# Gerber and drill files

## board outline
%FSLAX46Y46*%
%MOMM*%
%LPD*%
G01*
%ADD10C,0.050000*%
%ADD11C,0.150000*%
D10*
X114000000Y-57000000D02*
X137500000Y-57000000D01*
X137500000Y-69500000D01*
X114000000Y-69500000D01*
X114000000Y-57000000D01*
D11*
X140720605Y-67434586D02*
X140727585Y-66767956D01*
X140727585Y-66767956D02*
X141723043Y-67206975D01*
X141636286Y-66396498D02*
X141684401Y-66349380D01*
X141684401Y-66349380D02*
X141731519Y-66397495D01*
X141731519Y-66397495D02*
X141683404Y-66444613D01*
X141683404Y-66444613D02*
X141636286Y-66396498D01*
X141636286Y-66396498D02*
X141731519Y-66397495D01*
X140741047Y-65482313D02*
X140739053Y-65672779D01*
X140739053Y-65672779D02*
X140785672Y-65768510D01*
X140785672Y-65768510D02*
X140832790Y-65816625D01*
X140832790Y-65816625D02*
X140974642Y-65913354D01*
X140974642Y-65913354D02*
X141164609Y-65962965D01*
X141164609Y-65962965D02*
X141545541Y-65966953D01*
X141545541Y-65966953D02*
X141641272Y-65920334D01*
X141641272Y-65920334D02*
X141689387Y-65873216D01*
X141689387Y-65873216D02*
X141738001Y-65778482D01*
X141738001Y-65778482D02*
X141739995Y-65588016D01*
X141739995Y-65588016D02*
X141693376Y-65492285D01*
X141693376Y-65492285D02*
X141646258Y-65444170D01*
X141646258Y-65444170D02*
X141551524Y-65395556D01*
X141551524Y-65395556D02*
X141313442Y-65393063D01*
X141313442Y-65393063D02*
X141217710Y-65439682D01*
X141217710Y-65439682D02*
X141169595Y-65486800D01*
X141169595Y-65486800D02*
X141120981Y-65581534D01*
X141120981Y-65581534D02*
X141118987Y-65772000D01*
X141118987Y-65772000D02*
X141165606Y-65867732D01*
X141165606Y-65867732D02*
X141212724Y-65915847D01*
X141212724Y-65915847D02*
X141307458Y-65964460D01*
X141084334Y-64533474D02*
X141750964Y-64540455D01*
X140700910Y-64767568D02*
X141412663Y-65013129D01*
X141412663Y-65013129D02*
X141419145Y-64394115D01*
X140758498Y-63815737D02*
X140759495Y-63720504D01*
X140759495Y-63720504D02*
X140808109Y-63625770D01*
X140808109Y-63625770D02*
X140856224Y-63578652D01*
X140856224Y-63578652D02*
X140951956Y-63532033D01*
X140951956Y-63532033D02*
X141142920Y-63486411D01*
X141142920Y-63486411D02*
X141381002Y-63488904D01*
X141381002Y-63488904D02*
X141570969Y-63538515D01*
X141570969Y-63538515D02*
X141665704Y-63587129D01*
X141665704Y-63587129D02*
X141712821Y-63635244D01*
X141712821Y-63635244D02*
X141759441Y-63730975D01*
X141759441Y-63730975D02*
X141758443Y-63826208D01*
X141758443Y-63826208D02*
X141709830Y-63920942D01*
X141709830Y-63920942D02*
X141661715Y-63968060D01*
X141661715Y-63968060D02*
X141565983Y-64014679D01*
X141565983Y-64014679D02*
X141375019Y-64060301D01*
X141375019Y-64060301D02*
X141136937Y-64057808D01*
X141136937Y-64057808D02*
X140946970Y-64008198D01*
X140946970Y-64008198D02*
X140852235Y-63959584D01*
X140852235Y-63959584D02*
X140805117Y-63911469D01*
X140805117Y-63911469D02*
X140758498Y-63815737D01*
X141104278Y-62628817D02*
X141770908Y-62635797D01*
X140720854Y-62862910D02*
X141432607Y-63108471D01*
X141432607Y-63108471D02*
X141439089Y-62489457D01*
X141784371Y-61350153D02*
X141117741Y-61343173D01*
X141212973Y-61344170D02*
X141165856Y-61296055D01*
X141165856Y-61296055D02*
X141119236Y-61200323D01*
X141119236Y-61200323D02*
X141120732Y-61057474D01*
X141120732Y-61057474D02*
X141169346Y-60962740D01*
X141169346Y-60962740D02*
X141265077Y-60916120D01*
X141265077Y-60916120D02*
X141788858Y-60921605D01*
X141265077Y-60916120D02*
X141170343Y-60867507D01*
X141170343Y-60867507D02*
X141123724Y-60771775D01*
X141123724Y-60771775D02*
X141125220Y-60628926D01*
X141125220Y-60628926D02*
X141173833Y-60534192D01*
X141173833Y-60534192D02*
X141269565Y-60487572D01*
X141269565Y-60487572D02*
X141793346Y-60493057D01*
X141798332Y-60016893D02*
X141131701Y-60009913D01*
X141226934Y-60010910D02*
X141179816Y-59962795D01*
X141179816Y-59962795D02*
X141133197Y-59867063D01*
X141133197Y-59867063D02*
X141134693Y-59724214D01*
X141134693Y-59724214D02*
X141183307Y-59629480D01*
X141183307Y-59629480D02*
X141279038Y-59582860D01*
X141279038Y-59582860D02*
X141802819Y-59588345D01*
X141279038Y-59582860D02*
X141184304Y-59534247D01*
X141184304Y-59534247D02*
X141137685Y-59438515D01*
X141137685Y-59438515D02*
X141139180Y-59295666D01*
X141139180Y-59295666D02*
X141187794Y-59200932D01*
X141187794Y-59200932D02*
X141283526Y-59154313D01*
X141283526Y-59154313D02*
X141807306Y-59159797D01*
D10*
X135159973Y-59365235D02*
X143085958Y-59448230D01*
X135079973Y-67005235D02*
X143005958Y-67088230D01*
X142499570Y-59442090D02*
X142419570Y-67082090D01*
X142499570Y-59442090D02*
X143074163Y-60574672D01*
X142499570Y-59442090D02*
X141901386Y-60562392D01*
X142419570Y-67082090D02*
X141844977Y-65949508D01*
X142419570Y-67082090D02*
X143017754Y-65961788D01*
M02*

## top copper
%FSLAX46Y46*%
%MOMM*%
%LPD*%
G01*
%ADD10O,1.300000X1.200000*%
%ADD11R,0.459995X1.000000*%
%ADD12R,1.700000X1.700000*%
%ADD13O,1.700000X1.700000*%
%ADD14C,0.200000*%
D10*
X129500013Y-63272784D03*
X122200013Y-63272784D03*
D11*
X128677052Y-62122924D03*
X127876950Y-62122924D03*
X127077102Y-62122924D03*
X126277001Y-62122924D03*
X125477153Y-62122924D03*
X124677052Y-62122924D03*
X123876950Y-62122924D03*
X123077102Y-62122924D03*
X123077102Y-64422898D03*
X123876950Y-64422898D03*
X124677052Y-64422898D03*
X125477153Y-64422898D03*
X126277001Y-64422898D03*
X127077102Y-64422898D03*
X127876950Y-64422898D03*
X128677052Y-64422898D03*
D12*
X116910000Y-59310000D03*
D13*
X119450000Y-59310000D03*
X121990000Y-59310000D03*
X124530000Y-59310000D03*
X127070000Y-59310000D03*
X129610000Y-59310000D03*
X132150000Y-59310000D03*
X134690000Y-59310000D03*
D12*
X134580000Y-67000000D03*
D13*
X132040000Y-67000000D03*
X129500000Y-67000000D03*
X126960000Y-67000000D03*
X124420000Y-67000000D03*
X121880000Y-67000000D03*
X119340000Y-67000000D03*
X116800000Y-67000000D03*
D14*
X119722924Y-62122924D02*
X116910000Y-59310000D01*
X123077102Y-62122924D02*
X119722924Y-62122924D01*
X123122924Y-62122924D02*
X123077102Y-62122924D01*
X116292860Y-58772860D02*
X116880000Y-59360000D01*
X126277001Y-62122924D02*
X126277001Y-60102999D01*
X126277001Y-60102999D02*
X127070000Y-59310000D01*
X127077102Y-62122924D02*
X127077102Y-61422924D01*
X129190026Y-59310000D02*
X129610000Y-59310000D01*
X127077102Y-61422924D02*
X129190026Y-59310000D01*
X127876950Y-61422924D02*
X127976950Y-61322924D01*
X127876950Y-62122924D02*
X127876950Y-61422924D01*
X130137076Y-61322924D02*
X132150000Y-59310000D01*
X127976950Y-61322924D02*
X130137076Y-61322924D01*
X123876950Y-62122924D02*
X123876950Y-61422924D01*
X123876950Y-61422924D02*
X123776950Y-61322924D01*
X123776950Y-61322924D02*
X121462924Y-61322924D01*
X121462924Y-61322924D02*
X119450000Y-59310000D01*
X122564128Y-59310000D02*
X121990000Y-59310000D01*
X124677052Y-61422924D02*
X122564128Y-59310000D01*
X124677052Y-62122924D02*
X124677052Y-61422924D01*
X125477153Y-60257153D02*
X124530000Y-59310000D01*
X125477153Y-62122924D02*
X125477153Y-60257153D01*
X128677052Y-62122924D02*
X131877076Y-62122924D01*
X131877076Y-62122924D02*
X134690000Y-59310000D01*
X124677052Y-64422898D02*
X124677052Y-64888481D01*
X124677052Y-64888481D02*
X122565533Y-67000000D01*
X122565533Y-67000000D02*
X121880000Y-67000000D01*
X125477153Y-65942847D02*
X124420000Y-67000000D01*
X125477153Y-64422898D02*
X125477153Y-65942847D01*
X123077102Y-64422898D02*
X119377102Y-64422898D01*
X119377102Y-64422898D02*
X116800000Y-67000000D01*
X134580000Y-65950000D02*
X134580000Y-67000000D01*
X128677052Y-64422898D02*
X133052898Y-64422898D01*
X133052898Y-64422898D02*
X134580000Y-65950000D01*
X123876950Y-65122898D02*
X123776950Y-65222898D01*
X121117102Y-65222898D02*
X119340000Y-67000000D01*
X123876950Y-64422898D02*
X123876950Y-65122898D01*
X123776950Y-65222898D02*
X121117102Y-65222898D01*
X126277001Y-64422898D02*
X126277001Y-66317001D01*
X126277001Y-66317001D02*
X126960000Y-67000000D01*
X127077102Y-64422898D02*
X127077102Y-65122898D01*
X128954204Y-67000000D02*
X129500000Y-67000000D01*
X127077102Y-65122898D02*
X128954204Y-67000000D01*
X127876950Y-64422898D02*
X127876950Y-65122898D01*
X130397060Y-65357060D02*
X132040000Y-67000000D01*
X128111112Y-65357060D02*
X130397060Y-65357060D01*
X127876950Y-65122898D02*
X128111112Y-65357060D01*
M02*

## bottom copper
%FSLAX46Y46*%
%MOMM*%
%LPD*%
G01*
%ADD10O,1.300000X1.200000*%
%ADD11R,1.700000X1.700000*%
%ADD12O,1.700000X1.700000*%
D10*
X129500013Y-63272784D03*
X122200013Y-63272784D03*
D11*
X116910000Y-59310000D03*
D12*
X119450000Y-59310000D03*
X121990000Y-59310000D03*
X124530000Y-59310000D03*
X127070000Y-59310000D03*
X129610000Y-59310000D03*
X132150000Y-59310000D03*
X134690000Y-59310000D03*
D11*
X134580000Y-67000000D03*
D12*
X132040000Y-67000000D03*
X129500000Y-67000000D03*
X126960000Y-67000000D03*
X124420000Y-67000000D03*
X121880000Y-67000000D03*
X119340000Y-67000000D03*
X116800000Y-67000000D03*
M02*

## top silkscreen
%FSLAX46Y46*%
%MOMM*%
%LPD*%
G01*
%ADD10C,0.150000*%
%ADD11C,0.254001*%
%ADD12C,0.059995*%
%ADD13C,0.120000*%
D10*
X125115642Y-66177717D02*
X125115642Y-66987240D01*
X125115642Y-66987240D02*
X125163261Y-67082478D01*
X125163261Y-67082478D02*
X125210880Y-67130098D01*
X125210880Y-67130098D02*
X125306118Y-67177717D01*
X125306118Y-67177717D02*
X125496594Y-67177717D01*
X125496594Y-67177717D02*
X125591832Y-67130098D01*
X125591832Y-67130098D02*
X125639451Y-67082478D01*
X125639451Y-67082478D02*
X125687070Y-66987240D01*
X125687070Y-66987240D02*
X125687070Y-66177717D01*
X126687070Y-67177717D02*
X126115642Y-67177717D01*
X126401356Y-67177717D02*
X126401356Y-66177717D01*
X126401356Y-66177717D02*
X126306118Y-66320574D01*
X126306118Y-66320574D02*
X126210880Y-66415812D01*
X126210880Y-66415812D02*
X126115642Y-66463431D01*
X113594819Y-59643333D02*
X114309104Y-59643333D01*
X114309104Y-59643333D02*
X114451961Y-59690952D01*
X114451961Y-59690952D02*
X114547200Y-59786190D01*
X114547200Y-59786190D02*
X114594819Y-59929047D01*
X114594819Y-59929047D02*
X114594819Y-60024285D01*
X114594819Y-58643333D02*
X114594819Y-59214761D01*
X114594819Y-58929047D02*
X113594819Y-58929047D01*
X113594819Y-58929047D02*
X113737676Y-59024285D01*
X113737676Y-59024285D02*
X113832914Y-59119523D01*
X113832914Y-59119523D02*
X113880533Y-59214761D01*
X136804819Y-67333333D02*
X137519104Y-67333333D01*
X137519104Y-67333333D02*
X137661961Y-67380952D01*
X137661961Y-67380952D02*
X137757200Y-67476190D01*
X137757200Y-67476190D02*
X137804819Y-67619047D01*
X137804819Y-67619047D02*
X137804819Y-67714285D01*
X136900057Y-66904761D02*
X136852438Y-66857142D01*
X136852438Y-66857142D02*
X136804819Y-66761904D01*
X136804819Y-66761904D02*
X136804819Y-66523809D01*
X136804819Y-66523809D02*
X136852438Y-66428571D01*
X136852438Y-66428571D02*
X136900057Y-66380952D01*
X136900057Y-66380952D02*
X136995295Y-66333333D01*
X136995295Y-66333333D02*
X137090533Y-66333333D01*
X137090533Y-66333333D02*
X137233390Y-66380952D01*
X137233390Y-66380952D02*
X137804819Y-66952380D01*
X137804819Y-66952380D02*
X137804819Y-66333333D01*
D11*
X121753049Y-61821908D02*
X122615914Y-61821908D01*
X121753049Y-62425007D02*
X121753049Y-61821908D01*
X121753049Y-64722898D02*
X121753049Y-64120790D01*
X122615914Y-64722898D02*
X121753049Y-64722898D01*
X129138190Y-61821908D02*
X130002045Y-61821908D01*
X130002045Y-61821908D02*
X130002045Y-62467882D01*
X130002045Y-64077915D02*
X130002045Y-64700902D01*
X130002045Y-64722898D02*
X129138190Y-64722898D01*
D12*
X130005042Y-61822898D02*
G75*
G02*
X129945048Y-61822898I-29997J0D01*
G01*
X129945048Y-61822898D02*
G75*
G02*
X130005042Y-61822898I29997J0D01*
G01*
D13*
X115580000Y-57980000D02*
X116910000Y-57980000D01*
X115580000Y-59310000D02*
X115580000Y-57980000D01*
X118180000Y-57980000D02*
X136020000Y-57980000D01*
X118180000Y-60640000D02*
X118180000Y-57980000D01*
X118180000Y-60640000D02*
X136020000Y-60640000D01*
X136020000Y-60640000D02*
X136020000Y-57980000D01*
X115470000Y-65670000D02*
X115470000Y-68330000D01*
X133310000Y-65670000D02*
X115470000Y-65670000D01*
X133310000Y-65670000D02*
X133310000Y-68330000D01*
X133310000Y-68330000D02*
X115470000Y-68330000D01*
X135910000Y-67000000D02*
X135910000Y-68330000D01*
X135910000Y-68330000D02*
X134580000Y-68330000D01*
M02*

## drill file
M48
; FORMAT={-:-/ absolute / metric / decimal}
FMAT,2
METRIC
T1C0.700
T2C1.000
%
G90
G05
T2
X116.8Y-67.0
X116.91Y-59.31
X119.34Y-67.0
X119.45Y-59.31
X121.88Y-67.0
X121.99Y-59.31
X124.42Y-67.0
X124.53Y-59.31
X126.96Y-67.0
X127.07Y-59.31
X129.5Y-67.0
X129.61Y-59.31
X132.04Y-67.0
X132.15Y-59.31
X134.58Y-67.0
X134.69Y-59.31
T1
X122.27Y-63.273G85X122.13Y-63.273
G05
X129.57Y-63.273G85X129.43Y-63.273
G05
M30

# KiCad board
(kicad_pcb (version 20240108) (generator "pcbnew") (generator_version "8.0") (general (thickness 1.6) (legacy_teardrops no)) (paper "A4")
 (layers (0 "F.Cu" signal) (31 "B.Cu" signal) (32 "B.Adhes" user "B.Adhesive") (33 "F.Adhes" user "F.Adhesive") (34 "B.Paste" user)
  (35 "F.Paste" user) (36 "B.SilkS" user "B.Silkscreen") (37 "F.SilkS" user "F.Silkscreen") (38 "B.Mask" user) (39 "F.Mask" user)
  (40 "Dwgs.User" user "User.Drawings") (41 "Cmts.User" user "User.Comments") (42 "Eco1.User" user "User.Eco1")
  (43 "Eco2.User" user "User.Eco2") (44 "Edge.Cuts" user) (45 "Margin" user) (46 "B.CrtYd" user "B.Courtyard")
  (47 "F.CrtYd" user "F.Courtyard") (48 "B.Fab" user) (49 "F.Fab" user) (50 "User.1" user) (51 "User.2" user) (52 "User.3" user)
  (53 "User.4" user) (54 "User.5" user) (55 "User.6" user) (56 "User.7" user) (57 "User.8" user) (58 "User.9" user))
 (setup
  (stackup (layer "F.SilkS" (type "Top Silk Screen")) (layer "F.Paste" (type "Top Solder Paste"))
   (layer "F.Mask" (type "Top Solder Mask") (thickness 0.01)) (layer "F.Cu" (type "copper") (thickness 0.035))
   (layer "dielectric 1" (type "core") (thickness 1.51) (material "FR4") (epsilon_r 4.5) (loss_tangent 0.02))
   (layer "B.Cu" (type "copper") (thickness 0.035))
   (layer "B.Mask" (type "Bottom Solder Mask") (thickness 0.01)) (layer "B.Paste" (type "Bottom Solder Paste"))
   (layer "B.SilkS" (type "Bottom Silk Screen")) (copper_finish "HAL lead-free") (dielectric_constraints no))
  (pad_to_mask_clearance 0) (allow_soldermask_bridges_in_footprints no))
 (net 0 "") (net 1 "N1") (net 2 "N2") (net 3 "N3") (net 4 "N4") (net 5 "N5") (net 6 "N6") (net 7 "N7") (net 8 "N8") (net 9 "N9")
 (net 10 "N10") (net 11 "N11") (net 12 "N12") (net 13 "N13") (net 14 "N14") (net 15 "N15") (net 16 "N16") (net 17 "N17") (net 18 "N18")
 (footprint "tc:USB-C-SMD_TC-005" (layer "F.Cu") (at 125.850026 63.272911 180)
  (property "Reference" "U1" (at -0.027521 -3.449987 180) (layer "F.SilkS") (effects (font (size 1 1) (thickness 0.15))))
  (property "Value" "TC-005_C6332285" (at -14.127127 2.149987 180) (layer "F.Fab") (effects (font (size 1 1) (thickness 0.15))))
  (fp_line (start 4.096977 1.451003) (end 3.234112 1.451003) (stroke (width 0.254001) (type solid)) (layer "F.SilkS"))
  (fp_line (start 4.096977 0.847904) (end 4.096977 1.451003) (stroke (width 0.254001) (type solid)) (layer "F.SilkS"))
  (fp_line (start 4.096977 -1.449987) (end 4.096977 -0.847879) (stroke (width 0.254001) (type solid)) (layer "F.SilkS"))
  (fp_line (start 3.234112 -1.449987) (end 4.096977 -1.449987) (stroke (width 0.254001) (type solid)) (layer "F.SilkS"))
  (fp_line (start -3.288164 1.451003) (end -4.152019 1.451003) (stroke (width 0.254001) (type solid)) (layer "F.SilkS"))
  (fp_line (start -4.152019 1.451003) (end -4.152019 0.805029) (stroke (width 0.254001) (type solid)) (layer "F.SilkS"))
  (fp_line (start -4.152019 -0.805004) (end -4.152019 -1.427991) (stroke (width 0.254001) (type solid)) (layer "F.SilkS"))
  (fp_line (start -4.152019 -1.449987) (end -3.288164 -1.449987) (stroke (width 0.254001) (type solid)) (layer "F.SilkS"))
  (fp_circle (center -4.125019 1.450013) (end -4.095022 1.450013) (stroke (width 0.059995) (type solid)) (fill none) (layer "F.SilkS"))
  (pad "1" thru_hole oval (at -3.649987 0.000127 180) (size 1.3 1.2) (drill oval 0.840005 0.700025) (layers "*.Cu" "*.Mask")
   (remove_unused_layers no) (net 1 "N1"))
  (pad "2" thru_hole oval (at 3.650013 0.000127 180) (size 1.3 1.2) (drill oval 0.840005 0.700025) (layers "*.Cu" "*.Mask")
   (remove_unused_layers no) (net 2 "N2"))
  (pad "A1" smd rect (at -2.827026 1.149987 180) (size 0.459995 1) (layers "F.Cu" "F.Paste" "F.Mask") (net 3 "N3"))
  (pad "A4" smd rect (at -2.026924 1.149987 180) (size 0.459995 1) (layers "F.Cu" "F.Paste" "F.Mask") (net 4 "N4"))
  (pad "A5" smd rect (at -1.227076 1.149987 180) (size 0.459995 1) (layers "F.Cu" "F.Paste" "F.Mask") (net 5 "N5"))
  (pad "A6" smd rect (at -0.426975 1.149987 180) (size 0.459995 1) (layers "F.Cu" "F.Paste" "F.Mask") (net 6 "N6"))
  (pad "A7" smd rect (at 0.372873 1.149987 180) (size 0.459995 1) (layers "F.Cu" "F.Paste" "F.Mask") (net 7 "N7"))
  (pad "A8" smd rect (at 1.172974 1.149987 180) (size 0.459995 1) (layers "F.Cu" "F.Paste" "F.Mask") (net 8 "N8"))
  (pad "A9" smd rect (at 1.973076 1.149987 180) (size 0.459995 1) (layers "F.Cu" "F.Paste" "F.Mask") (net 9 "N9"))
  (pad "A12" smd rect (at 2.772924 1.149987 180) (size 0.459995 1) (layers "F.Cu" "F.Paste" "F.Mask") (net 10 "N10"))
  (pad "B1" smd rect (at 2.772924 -1.149987 180) (size 0.459995 1) (layers "F.Cu" "F.Paste" "F.Mask") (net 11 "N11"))
  (pad "B4" smd rect (at 1.973076 -1.149987 180) (size 0.459995 1) (layers "F.Cu" "F.Paste" "F.Mask") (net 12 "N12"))
  (pad "B5" smd rect (at 1.172974 -1.149987 180) (size 0.459995 1) (layers "F.Cu" "F.Paste" "F.Mask") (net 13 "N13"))
  (pad "B6" smd rect (at 0.372873 -1.149987 180) (size 0.459995 1) (layers "F.Cu" "F.Paste" "F.Mask") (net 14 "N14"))
  (pad "B7" smd rect (at -0.426975 -1.149987 180) (size 0.459995 1) (layers "F.Cu" "F.Paste" "F.Mask") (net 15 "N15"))
  (pad "B8" smd rect (at -1.227076 -1.149987 180) (size 0.459995 1) (layers "F.Cu" "F.Paste" "F.Mask") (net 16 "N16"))
  (pad "B9" smd rect (at -2.026924 -1.149987 180) (size 0.459995 1) (layers "F.Cu" "F.Paste" "F.Mask") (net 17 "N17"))
  (pad "B12" smd rect (at -2.827026 -1.149987 180) (size 0.459995 1) (layers "F.Cu" "F.Paste" "F.Mask") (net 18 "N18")))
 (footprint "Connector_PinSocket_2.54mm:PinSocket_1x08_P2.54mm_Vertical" (layer "F.Cu") (at 116.91 59.31 90)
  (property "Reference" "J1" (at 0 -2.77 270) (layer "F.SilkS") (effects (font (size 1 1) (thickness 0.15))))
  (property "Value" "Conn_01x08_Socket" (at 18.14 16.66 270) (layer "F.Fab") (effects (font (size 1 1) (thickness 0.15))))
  (fp_line (start 1.33 -1.33) (end 1.33 0) (stroke (width 0.12) (type solid)) (layer "F.SilkS"))
  (fp_line (start 0 -1.33) (end 1.33 -1.33) (stroke (width 0.12) (type solid)) (layer "F.SilkS"))
  (fp_line (start 1.33 1.27) (end 1.33 19.11) (stroke (width 0.12) (type solid)) (layer "F.SilkS"))
  (fp_line (start -1.33 1.27) (end 1.33 1.27) (stroke (width 0.12) (type solid)) (layer "F.SilkS"))
  (fp_line (start -1.33 1.27) (end -1.33 19.11) (stroke (width 0.12) (type solid)) (layer "F.SilkS"))
  (fp_line (start -1.33 19.11) (end 1.33 19.11) (stroke (width 0.12) (type solid)) (layer "F.SilkS"))
  (pad "1" thru_hole rect (at 0 0 90) (size 1.7 1.7) (drill 1) (layers "*.Cu" "*.Mask") (remove_unused_layers no) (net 10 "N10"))
  (pad "2" thru_hole oval (at 0 2.54 90) (size 1.7 1.7) (drill 1) (layers "*.Cu" "*.Mask") (remove_unused_layers no) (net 9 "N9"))
  (pad "3" thru_hole oval (at 0 5.08 90) (size 1.7 1.7) (drill 1) (layers "*.Cu" "*.Mask") (remove_unused_layers no) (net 8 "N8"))
  (pad "4" thru_hole oval (at 0 7.62 90) (size 1.7 1.7) (drill 1) (layers "*.Cu" "*.Mask") (remove_unused_layers no) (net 7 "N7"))
  (pad "5" thru_hole oval (at 0 10.16 90) (size 1.7 1.7) (drill 1) (layers "*.Cu" "*.Mask") (remove_unused_layers no) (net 6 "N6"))
  (pad "6" thru_hole oval (at 0 12.7 90) (size 1.7 1.7) (drill 1) (layers "*.Cu" "*.Mask") (remove_unused_layers no) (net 5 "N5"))
  (pad "7" thru_hole oval (at 0 15.24 90) (size 1.7 1.7) (drill 1) (layers "*.Cu" "*.Mask") (remove_unused_layers no) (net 4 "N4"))
  (pad "8" thru_hole oval (at 0 17.78 90) (size 1.7 1.7) (drill 1) (layers "*.Cu" "*.Mask") (remove_unused_layers no) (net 3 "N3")))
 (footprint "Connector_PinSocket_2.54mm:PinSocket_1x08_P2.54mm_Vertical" (layer "F.Cu") (at 134.58 67 -90)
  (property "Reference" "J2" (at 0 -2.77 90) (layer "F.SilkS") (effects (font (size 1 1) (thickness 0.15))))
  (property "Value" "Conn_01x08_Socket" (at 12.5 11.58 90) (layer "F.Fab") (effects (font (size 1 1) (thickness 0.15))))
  (fp_line (start -1.33 19.11) (end 1.33 19.11) (stroke (width 0.12) (type solid)) (layer "F.SilkS"))
  (fp_line (start -1.33 1.27) (end -1.33 19.11) (stroke (width 0.12) (type solid)) (layer "F.SilkS"))
  (fp_line (start -1.33 1.27) (end 1.33 1.27) (stroke (width 0.12) (type solid)) (layer "F.SilkS"))
  (fp_line (start 1.33 1.27) (end 1.33 19.11) (stroke (width 0.12) (type solid)) (layer "F.SilkS"))
  (fp_line (start 0 -1.33) (end 1.33 -1.33) (stroke (width 0.12) (type solid)) (layer "F.SilkS"))
  (fp_line (start 1.33 -1.33) (end 1.33 0) (stroke (width 0.12) (type solid)) (layer "F.SilkS"))
  (pad "1" thru_hole rect (at 0 0 270) (size 1.7 1.7) (drill 1) (layers "*.Cu" "*.Mask") (remove_unused_layers no) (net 18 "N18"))
  (pad "2" thru_hole oval (at 0 2.54 270) (size 1.7 1.7) (drill 1) (layers "*.Cu" "*.Mask") (remove_unused_layers no) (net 17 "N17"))
  (pad "3" thru_hole oval (at 0 5.08 270) (size 1.7 1.7) (drill 1) (layers "*.Cu" "*.Mask") (remove_unused_layers no) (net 16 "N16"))
  (pad "4" thru_hole oval (at 0 7.62 270) (size 1.7 1.7) (drill 1) (layers "*.Cu" "*.Mask") (remove_unused_layers no) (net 15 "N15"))
  (pad "5" thru_hole oval (at 0 10.16 270) (size 1.7 1.7) (drill 1) (layers "*.Cu" "*.Mask") (remove_unused_layers no) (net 14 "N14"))
  (pad "6" thru_hole oval (at 0 12.7 270) (size 1.7 1.7) (drill 1) (layers "*.Cu" "*.Mask") (remove_unused_layers no) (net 13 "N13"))
  (pad "7" thru_hole oval (at 0 15.24 270) (size 1.7 1.7) (drill 1) (layers "*.Cu" "*.Mask") (remove_unused_layers no) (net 12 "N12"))
  (pad "8" thru_hole oval (at 0 17.78 270) (size 1.7 1.7) (drill 1) (layers "*.Cu" "*.Mask") (remove_unused_layers no) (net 11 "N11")))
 (gr_rect (start 114 57) (end 137.5 69.5) (stroke (width 0.05) (type default)) (fill none) (layer "Edge.Cuts"))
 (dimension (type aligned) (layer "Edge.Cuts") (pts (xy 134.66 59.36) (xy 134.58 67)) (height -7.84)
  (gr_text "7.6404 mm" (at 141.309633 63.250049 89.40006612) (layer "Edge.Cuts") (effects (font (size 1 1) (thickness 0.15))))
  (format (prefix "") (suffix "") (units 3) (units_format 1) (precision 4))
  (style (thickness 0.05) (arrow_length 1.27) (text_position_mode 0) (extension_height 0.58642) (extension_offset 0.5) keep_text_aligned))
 (segment (start 119.722924 62.122924) (end 116.91 59.31) (width 0.2) (layer "F.Cu") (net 10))
 (segment (start 123.077102 62.122924) (end 119.722924 62.122924) (width 0.2) (layer "F.Cu") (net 10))
 (segment (start 123.122924 62.122924) (end 123.077102 62.122924) (width 0.2) (layer "F.Cu") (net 10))
 (segment (start 116.29286 58.77286) (end 116.88 59.36) (width 0.2) (layer "F.Cu") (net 10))
 (segment (start 126.277001 62.122924) (end 126.277001 60.102999) (width 0.2) (layer "F.Cu") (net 6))
 (segment (start 126.277001 60.102999) (end 127.07 59.31) (width 0.2) (layer "F.Cu") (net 6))
 (segment (start 127.077102 62.122924) (end 127.077102 61.422924) (width 0.2) (layer "F.Cu") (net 5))
 (segment (start 129.190026 59.31) (end 129.61 59.31) (width 0.2) (layer "F.Cu") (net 5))
 (segment (start 127.077102 61.422924) (end 129.190026 59.31) (width 0.2) (layer "F.Cu") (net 5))
 (segment (start 127.87695 61.422924) (end 127.97695 61.322924) (width 0.2) (layer "F.Cu") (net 4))
 (segment (start 127.87695 62.122924) (end 127.87695 61.422924) (width 0.2) (layer "F.Cu") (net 4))
 (segment (start 130.137076 61.322924) (end 132.15 59.31) (width 0.2) (layer "F.Cu") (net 4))
 (segment (start 127.97695 61.322924) (end 130.137076 61.322924) (width 0.2) (layer "F.Cu") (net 4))
 (segment (start 123.87695 62.122924) (end 123.87695 61.422924) (width 0.2) (layer "F.Cu") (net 9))
 (segment (start 123.87695 61.422924) (end 123.77695 61.322924) (width 0.2) (layer "F.Cu") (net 9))
 (segment (start 123.77695 61.322924) (end 121.462924 61.322924) (width 0.2) (layer "F.Cu") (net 9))
 (segment (start 121.462924 61.322924) (end 119.45 59.31) (width 0.2) (layer "F.Cu") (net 9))
 (segment (start 122.564128 59.31) (end 121.99 59.31) (width 0.2) (layer "F.Cu") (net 8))
 (segment (start 124.677052 61.422924) (end 122.564128 59.31) (width 0.2) (layer "F.Cu") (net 8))
 (segment (start 124.677052 62.122924) (end 124.677052 61.422924) (width 0.2) (layer "F.Cu") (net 8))
 (segment (start 125.477153 60.257153) (end 124.53 59.31) (width 0.2) (layer "F.Cu") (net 7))
 (segment (start 125.477153 62.122924) (end 125.477153 60.257153) (width 0.2) (layer "F.Cu") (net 7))
 (segment (start 128.677052 62.122924) (end 131.877076 62.122924) (width 0.2) (layer "F.Cu") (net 3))
 (segment (start 131.877076 62.122924) (end 134.69 59.31) (width 0.2) (layer "F.Cu") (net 3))
 (segment (start 124.677052 64.422898) (end 124.677052 64.888481) (width 0.2) (layer "F.Cu") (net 13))
 (segment (start 124.677052 64.888481) (end 122.565533 67) (width 0.2) (layer "F.Cu") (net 13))
 (segment (start 122.565533 67) (end 121.88 67) (width 0.2) (layer "F.Cu") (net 13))
 (segment (start 125.477153 65.942847) (end 124.42 67) (width 0.2) (layer "F.Cu") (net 14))
 (segment (start 125.477153 64.422898) (end 125.477153 65.942847) (width 0.2) (layer "F.Cu") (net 14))
 (segment (start 123.077102 64.422898) (end 119.377102 64.422898) (width 0.2) (layer "F.Cu") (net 11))
 (segment (start 119.377102 64.422898) (end 116.8 67) (width 0.2) (layer "F.Cu") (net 11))
 (segment (start 134.58 65.95) (end 134.58 67) (width 0.2) (layer "F.Cu") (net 18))
 (segment (start 128.677052 64.422898) (end 133.052898 64.422898) (width 0.2) (layer "F.Cu") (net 18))
 (segment (start 133.052898 64.422898) (end 134.58 65.95) (width 0.2) (layer "F.Cu") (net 18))
 (segment (start 123.87695 65.122898) (end 123.77695 65.222898) (width 0.2) (layer "F.Cu") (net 12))
 (segment (start 121.117102 65.222898) (end 119.34 67) (width 0.2) (layer "F.Cu") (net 12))
 (segment (start 123.87695 64.422898) (end 123.87695 65.122898) (width 0.2) (layer "F.Cu") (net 12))
 (segment (start 123.77695 65.222898) (end 121.117102 65.222898) (width 0.2) (layer "F.Cu") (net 12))
 (segment (start 126.277001 64.422898) (end 126.277001 66.317001) (width 0.2) (layer "F.Cu") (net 15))
 (segment (start 126.277001 66.317001) (end 126.96 67) (width 0.2) (layer "F.Cu") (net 15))
 (segment (start 127.077102 64.422898) (end 127.077102 65.122898) (width 0.2) (layer "F.Cu") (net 16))
 (segment (start 128.954204 67) (end 129.5 67) (width 0.2) (layer "F.Cu") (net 16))
 (segment (start 127.077102 65.122898) (end 128.954204 67) (width 0.2) (layer "F.Cu") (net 16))
 (segment (start 127.87695 64.422898) (end 127.87695 65.122898) (width 0.2) (layer "F.Cu") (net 17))
 (segment (start 130.39706 65.35706) (end 132.04 67) (width 0.2) (layer "F.Cu") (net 17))
 (segment (start 128.111112 65.35706) (end 130.39706 65.35706) (width 0.2) (layer "F.Cu") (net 17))
 (segment (start 127.87695 65.122898) (end 128.111112 65.35706) (width 0.2) (layer "F.Cu") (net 17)))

